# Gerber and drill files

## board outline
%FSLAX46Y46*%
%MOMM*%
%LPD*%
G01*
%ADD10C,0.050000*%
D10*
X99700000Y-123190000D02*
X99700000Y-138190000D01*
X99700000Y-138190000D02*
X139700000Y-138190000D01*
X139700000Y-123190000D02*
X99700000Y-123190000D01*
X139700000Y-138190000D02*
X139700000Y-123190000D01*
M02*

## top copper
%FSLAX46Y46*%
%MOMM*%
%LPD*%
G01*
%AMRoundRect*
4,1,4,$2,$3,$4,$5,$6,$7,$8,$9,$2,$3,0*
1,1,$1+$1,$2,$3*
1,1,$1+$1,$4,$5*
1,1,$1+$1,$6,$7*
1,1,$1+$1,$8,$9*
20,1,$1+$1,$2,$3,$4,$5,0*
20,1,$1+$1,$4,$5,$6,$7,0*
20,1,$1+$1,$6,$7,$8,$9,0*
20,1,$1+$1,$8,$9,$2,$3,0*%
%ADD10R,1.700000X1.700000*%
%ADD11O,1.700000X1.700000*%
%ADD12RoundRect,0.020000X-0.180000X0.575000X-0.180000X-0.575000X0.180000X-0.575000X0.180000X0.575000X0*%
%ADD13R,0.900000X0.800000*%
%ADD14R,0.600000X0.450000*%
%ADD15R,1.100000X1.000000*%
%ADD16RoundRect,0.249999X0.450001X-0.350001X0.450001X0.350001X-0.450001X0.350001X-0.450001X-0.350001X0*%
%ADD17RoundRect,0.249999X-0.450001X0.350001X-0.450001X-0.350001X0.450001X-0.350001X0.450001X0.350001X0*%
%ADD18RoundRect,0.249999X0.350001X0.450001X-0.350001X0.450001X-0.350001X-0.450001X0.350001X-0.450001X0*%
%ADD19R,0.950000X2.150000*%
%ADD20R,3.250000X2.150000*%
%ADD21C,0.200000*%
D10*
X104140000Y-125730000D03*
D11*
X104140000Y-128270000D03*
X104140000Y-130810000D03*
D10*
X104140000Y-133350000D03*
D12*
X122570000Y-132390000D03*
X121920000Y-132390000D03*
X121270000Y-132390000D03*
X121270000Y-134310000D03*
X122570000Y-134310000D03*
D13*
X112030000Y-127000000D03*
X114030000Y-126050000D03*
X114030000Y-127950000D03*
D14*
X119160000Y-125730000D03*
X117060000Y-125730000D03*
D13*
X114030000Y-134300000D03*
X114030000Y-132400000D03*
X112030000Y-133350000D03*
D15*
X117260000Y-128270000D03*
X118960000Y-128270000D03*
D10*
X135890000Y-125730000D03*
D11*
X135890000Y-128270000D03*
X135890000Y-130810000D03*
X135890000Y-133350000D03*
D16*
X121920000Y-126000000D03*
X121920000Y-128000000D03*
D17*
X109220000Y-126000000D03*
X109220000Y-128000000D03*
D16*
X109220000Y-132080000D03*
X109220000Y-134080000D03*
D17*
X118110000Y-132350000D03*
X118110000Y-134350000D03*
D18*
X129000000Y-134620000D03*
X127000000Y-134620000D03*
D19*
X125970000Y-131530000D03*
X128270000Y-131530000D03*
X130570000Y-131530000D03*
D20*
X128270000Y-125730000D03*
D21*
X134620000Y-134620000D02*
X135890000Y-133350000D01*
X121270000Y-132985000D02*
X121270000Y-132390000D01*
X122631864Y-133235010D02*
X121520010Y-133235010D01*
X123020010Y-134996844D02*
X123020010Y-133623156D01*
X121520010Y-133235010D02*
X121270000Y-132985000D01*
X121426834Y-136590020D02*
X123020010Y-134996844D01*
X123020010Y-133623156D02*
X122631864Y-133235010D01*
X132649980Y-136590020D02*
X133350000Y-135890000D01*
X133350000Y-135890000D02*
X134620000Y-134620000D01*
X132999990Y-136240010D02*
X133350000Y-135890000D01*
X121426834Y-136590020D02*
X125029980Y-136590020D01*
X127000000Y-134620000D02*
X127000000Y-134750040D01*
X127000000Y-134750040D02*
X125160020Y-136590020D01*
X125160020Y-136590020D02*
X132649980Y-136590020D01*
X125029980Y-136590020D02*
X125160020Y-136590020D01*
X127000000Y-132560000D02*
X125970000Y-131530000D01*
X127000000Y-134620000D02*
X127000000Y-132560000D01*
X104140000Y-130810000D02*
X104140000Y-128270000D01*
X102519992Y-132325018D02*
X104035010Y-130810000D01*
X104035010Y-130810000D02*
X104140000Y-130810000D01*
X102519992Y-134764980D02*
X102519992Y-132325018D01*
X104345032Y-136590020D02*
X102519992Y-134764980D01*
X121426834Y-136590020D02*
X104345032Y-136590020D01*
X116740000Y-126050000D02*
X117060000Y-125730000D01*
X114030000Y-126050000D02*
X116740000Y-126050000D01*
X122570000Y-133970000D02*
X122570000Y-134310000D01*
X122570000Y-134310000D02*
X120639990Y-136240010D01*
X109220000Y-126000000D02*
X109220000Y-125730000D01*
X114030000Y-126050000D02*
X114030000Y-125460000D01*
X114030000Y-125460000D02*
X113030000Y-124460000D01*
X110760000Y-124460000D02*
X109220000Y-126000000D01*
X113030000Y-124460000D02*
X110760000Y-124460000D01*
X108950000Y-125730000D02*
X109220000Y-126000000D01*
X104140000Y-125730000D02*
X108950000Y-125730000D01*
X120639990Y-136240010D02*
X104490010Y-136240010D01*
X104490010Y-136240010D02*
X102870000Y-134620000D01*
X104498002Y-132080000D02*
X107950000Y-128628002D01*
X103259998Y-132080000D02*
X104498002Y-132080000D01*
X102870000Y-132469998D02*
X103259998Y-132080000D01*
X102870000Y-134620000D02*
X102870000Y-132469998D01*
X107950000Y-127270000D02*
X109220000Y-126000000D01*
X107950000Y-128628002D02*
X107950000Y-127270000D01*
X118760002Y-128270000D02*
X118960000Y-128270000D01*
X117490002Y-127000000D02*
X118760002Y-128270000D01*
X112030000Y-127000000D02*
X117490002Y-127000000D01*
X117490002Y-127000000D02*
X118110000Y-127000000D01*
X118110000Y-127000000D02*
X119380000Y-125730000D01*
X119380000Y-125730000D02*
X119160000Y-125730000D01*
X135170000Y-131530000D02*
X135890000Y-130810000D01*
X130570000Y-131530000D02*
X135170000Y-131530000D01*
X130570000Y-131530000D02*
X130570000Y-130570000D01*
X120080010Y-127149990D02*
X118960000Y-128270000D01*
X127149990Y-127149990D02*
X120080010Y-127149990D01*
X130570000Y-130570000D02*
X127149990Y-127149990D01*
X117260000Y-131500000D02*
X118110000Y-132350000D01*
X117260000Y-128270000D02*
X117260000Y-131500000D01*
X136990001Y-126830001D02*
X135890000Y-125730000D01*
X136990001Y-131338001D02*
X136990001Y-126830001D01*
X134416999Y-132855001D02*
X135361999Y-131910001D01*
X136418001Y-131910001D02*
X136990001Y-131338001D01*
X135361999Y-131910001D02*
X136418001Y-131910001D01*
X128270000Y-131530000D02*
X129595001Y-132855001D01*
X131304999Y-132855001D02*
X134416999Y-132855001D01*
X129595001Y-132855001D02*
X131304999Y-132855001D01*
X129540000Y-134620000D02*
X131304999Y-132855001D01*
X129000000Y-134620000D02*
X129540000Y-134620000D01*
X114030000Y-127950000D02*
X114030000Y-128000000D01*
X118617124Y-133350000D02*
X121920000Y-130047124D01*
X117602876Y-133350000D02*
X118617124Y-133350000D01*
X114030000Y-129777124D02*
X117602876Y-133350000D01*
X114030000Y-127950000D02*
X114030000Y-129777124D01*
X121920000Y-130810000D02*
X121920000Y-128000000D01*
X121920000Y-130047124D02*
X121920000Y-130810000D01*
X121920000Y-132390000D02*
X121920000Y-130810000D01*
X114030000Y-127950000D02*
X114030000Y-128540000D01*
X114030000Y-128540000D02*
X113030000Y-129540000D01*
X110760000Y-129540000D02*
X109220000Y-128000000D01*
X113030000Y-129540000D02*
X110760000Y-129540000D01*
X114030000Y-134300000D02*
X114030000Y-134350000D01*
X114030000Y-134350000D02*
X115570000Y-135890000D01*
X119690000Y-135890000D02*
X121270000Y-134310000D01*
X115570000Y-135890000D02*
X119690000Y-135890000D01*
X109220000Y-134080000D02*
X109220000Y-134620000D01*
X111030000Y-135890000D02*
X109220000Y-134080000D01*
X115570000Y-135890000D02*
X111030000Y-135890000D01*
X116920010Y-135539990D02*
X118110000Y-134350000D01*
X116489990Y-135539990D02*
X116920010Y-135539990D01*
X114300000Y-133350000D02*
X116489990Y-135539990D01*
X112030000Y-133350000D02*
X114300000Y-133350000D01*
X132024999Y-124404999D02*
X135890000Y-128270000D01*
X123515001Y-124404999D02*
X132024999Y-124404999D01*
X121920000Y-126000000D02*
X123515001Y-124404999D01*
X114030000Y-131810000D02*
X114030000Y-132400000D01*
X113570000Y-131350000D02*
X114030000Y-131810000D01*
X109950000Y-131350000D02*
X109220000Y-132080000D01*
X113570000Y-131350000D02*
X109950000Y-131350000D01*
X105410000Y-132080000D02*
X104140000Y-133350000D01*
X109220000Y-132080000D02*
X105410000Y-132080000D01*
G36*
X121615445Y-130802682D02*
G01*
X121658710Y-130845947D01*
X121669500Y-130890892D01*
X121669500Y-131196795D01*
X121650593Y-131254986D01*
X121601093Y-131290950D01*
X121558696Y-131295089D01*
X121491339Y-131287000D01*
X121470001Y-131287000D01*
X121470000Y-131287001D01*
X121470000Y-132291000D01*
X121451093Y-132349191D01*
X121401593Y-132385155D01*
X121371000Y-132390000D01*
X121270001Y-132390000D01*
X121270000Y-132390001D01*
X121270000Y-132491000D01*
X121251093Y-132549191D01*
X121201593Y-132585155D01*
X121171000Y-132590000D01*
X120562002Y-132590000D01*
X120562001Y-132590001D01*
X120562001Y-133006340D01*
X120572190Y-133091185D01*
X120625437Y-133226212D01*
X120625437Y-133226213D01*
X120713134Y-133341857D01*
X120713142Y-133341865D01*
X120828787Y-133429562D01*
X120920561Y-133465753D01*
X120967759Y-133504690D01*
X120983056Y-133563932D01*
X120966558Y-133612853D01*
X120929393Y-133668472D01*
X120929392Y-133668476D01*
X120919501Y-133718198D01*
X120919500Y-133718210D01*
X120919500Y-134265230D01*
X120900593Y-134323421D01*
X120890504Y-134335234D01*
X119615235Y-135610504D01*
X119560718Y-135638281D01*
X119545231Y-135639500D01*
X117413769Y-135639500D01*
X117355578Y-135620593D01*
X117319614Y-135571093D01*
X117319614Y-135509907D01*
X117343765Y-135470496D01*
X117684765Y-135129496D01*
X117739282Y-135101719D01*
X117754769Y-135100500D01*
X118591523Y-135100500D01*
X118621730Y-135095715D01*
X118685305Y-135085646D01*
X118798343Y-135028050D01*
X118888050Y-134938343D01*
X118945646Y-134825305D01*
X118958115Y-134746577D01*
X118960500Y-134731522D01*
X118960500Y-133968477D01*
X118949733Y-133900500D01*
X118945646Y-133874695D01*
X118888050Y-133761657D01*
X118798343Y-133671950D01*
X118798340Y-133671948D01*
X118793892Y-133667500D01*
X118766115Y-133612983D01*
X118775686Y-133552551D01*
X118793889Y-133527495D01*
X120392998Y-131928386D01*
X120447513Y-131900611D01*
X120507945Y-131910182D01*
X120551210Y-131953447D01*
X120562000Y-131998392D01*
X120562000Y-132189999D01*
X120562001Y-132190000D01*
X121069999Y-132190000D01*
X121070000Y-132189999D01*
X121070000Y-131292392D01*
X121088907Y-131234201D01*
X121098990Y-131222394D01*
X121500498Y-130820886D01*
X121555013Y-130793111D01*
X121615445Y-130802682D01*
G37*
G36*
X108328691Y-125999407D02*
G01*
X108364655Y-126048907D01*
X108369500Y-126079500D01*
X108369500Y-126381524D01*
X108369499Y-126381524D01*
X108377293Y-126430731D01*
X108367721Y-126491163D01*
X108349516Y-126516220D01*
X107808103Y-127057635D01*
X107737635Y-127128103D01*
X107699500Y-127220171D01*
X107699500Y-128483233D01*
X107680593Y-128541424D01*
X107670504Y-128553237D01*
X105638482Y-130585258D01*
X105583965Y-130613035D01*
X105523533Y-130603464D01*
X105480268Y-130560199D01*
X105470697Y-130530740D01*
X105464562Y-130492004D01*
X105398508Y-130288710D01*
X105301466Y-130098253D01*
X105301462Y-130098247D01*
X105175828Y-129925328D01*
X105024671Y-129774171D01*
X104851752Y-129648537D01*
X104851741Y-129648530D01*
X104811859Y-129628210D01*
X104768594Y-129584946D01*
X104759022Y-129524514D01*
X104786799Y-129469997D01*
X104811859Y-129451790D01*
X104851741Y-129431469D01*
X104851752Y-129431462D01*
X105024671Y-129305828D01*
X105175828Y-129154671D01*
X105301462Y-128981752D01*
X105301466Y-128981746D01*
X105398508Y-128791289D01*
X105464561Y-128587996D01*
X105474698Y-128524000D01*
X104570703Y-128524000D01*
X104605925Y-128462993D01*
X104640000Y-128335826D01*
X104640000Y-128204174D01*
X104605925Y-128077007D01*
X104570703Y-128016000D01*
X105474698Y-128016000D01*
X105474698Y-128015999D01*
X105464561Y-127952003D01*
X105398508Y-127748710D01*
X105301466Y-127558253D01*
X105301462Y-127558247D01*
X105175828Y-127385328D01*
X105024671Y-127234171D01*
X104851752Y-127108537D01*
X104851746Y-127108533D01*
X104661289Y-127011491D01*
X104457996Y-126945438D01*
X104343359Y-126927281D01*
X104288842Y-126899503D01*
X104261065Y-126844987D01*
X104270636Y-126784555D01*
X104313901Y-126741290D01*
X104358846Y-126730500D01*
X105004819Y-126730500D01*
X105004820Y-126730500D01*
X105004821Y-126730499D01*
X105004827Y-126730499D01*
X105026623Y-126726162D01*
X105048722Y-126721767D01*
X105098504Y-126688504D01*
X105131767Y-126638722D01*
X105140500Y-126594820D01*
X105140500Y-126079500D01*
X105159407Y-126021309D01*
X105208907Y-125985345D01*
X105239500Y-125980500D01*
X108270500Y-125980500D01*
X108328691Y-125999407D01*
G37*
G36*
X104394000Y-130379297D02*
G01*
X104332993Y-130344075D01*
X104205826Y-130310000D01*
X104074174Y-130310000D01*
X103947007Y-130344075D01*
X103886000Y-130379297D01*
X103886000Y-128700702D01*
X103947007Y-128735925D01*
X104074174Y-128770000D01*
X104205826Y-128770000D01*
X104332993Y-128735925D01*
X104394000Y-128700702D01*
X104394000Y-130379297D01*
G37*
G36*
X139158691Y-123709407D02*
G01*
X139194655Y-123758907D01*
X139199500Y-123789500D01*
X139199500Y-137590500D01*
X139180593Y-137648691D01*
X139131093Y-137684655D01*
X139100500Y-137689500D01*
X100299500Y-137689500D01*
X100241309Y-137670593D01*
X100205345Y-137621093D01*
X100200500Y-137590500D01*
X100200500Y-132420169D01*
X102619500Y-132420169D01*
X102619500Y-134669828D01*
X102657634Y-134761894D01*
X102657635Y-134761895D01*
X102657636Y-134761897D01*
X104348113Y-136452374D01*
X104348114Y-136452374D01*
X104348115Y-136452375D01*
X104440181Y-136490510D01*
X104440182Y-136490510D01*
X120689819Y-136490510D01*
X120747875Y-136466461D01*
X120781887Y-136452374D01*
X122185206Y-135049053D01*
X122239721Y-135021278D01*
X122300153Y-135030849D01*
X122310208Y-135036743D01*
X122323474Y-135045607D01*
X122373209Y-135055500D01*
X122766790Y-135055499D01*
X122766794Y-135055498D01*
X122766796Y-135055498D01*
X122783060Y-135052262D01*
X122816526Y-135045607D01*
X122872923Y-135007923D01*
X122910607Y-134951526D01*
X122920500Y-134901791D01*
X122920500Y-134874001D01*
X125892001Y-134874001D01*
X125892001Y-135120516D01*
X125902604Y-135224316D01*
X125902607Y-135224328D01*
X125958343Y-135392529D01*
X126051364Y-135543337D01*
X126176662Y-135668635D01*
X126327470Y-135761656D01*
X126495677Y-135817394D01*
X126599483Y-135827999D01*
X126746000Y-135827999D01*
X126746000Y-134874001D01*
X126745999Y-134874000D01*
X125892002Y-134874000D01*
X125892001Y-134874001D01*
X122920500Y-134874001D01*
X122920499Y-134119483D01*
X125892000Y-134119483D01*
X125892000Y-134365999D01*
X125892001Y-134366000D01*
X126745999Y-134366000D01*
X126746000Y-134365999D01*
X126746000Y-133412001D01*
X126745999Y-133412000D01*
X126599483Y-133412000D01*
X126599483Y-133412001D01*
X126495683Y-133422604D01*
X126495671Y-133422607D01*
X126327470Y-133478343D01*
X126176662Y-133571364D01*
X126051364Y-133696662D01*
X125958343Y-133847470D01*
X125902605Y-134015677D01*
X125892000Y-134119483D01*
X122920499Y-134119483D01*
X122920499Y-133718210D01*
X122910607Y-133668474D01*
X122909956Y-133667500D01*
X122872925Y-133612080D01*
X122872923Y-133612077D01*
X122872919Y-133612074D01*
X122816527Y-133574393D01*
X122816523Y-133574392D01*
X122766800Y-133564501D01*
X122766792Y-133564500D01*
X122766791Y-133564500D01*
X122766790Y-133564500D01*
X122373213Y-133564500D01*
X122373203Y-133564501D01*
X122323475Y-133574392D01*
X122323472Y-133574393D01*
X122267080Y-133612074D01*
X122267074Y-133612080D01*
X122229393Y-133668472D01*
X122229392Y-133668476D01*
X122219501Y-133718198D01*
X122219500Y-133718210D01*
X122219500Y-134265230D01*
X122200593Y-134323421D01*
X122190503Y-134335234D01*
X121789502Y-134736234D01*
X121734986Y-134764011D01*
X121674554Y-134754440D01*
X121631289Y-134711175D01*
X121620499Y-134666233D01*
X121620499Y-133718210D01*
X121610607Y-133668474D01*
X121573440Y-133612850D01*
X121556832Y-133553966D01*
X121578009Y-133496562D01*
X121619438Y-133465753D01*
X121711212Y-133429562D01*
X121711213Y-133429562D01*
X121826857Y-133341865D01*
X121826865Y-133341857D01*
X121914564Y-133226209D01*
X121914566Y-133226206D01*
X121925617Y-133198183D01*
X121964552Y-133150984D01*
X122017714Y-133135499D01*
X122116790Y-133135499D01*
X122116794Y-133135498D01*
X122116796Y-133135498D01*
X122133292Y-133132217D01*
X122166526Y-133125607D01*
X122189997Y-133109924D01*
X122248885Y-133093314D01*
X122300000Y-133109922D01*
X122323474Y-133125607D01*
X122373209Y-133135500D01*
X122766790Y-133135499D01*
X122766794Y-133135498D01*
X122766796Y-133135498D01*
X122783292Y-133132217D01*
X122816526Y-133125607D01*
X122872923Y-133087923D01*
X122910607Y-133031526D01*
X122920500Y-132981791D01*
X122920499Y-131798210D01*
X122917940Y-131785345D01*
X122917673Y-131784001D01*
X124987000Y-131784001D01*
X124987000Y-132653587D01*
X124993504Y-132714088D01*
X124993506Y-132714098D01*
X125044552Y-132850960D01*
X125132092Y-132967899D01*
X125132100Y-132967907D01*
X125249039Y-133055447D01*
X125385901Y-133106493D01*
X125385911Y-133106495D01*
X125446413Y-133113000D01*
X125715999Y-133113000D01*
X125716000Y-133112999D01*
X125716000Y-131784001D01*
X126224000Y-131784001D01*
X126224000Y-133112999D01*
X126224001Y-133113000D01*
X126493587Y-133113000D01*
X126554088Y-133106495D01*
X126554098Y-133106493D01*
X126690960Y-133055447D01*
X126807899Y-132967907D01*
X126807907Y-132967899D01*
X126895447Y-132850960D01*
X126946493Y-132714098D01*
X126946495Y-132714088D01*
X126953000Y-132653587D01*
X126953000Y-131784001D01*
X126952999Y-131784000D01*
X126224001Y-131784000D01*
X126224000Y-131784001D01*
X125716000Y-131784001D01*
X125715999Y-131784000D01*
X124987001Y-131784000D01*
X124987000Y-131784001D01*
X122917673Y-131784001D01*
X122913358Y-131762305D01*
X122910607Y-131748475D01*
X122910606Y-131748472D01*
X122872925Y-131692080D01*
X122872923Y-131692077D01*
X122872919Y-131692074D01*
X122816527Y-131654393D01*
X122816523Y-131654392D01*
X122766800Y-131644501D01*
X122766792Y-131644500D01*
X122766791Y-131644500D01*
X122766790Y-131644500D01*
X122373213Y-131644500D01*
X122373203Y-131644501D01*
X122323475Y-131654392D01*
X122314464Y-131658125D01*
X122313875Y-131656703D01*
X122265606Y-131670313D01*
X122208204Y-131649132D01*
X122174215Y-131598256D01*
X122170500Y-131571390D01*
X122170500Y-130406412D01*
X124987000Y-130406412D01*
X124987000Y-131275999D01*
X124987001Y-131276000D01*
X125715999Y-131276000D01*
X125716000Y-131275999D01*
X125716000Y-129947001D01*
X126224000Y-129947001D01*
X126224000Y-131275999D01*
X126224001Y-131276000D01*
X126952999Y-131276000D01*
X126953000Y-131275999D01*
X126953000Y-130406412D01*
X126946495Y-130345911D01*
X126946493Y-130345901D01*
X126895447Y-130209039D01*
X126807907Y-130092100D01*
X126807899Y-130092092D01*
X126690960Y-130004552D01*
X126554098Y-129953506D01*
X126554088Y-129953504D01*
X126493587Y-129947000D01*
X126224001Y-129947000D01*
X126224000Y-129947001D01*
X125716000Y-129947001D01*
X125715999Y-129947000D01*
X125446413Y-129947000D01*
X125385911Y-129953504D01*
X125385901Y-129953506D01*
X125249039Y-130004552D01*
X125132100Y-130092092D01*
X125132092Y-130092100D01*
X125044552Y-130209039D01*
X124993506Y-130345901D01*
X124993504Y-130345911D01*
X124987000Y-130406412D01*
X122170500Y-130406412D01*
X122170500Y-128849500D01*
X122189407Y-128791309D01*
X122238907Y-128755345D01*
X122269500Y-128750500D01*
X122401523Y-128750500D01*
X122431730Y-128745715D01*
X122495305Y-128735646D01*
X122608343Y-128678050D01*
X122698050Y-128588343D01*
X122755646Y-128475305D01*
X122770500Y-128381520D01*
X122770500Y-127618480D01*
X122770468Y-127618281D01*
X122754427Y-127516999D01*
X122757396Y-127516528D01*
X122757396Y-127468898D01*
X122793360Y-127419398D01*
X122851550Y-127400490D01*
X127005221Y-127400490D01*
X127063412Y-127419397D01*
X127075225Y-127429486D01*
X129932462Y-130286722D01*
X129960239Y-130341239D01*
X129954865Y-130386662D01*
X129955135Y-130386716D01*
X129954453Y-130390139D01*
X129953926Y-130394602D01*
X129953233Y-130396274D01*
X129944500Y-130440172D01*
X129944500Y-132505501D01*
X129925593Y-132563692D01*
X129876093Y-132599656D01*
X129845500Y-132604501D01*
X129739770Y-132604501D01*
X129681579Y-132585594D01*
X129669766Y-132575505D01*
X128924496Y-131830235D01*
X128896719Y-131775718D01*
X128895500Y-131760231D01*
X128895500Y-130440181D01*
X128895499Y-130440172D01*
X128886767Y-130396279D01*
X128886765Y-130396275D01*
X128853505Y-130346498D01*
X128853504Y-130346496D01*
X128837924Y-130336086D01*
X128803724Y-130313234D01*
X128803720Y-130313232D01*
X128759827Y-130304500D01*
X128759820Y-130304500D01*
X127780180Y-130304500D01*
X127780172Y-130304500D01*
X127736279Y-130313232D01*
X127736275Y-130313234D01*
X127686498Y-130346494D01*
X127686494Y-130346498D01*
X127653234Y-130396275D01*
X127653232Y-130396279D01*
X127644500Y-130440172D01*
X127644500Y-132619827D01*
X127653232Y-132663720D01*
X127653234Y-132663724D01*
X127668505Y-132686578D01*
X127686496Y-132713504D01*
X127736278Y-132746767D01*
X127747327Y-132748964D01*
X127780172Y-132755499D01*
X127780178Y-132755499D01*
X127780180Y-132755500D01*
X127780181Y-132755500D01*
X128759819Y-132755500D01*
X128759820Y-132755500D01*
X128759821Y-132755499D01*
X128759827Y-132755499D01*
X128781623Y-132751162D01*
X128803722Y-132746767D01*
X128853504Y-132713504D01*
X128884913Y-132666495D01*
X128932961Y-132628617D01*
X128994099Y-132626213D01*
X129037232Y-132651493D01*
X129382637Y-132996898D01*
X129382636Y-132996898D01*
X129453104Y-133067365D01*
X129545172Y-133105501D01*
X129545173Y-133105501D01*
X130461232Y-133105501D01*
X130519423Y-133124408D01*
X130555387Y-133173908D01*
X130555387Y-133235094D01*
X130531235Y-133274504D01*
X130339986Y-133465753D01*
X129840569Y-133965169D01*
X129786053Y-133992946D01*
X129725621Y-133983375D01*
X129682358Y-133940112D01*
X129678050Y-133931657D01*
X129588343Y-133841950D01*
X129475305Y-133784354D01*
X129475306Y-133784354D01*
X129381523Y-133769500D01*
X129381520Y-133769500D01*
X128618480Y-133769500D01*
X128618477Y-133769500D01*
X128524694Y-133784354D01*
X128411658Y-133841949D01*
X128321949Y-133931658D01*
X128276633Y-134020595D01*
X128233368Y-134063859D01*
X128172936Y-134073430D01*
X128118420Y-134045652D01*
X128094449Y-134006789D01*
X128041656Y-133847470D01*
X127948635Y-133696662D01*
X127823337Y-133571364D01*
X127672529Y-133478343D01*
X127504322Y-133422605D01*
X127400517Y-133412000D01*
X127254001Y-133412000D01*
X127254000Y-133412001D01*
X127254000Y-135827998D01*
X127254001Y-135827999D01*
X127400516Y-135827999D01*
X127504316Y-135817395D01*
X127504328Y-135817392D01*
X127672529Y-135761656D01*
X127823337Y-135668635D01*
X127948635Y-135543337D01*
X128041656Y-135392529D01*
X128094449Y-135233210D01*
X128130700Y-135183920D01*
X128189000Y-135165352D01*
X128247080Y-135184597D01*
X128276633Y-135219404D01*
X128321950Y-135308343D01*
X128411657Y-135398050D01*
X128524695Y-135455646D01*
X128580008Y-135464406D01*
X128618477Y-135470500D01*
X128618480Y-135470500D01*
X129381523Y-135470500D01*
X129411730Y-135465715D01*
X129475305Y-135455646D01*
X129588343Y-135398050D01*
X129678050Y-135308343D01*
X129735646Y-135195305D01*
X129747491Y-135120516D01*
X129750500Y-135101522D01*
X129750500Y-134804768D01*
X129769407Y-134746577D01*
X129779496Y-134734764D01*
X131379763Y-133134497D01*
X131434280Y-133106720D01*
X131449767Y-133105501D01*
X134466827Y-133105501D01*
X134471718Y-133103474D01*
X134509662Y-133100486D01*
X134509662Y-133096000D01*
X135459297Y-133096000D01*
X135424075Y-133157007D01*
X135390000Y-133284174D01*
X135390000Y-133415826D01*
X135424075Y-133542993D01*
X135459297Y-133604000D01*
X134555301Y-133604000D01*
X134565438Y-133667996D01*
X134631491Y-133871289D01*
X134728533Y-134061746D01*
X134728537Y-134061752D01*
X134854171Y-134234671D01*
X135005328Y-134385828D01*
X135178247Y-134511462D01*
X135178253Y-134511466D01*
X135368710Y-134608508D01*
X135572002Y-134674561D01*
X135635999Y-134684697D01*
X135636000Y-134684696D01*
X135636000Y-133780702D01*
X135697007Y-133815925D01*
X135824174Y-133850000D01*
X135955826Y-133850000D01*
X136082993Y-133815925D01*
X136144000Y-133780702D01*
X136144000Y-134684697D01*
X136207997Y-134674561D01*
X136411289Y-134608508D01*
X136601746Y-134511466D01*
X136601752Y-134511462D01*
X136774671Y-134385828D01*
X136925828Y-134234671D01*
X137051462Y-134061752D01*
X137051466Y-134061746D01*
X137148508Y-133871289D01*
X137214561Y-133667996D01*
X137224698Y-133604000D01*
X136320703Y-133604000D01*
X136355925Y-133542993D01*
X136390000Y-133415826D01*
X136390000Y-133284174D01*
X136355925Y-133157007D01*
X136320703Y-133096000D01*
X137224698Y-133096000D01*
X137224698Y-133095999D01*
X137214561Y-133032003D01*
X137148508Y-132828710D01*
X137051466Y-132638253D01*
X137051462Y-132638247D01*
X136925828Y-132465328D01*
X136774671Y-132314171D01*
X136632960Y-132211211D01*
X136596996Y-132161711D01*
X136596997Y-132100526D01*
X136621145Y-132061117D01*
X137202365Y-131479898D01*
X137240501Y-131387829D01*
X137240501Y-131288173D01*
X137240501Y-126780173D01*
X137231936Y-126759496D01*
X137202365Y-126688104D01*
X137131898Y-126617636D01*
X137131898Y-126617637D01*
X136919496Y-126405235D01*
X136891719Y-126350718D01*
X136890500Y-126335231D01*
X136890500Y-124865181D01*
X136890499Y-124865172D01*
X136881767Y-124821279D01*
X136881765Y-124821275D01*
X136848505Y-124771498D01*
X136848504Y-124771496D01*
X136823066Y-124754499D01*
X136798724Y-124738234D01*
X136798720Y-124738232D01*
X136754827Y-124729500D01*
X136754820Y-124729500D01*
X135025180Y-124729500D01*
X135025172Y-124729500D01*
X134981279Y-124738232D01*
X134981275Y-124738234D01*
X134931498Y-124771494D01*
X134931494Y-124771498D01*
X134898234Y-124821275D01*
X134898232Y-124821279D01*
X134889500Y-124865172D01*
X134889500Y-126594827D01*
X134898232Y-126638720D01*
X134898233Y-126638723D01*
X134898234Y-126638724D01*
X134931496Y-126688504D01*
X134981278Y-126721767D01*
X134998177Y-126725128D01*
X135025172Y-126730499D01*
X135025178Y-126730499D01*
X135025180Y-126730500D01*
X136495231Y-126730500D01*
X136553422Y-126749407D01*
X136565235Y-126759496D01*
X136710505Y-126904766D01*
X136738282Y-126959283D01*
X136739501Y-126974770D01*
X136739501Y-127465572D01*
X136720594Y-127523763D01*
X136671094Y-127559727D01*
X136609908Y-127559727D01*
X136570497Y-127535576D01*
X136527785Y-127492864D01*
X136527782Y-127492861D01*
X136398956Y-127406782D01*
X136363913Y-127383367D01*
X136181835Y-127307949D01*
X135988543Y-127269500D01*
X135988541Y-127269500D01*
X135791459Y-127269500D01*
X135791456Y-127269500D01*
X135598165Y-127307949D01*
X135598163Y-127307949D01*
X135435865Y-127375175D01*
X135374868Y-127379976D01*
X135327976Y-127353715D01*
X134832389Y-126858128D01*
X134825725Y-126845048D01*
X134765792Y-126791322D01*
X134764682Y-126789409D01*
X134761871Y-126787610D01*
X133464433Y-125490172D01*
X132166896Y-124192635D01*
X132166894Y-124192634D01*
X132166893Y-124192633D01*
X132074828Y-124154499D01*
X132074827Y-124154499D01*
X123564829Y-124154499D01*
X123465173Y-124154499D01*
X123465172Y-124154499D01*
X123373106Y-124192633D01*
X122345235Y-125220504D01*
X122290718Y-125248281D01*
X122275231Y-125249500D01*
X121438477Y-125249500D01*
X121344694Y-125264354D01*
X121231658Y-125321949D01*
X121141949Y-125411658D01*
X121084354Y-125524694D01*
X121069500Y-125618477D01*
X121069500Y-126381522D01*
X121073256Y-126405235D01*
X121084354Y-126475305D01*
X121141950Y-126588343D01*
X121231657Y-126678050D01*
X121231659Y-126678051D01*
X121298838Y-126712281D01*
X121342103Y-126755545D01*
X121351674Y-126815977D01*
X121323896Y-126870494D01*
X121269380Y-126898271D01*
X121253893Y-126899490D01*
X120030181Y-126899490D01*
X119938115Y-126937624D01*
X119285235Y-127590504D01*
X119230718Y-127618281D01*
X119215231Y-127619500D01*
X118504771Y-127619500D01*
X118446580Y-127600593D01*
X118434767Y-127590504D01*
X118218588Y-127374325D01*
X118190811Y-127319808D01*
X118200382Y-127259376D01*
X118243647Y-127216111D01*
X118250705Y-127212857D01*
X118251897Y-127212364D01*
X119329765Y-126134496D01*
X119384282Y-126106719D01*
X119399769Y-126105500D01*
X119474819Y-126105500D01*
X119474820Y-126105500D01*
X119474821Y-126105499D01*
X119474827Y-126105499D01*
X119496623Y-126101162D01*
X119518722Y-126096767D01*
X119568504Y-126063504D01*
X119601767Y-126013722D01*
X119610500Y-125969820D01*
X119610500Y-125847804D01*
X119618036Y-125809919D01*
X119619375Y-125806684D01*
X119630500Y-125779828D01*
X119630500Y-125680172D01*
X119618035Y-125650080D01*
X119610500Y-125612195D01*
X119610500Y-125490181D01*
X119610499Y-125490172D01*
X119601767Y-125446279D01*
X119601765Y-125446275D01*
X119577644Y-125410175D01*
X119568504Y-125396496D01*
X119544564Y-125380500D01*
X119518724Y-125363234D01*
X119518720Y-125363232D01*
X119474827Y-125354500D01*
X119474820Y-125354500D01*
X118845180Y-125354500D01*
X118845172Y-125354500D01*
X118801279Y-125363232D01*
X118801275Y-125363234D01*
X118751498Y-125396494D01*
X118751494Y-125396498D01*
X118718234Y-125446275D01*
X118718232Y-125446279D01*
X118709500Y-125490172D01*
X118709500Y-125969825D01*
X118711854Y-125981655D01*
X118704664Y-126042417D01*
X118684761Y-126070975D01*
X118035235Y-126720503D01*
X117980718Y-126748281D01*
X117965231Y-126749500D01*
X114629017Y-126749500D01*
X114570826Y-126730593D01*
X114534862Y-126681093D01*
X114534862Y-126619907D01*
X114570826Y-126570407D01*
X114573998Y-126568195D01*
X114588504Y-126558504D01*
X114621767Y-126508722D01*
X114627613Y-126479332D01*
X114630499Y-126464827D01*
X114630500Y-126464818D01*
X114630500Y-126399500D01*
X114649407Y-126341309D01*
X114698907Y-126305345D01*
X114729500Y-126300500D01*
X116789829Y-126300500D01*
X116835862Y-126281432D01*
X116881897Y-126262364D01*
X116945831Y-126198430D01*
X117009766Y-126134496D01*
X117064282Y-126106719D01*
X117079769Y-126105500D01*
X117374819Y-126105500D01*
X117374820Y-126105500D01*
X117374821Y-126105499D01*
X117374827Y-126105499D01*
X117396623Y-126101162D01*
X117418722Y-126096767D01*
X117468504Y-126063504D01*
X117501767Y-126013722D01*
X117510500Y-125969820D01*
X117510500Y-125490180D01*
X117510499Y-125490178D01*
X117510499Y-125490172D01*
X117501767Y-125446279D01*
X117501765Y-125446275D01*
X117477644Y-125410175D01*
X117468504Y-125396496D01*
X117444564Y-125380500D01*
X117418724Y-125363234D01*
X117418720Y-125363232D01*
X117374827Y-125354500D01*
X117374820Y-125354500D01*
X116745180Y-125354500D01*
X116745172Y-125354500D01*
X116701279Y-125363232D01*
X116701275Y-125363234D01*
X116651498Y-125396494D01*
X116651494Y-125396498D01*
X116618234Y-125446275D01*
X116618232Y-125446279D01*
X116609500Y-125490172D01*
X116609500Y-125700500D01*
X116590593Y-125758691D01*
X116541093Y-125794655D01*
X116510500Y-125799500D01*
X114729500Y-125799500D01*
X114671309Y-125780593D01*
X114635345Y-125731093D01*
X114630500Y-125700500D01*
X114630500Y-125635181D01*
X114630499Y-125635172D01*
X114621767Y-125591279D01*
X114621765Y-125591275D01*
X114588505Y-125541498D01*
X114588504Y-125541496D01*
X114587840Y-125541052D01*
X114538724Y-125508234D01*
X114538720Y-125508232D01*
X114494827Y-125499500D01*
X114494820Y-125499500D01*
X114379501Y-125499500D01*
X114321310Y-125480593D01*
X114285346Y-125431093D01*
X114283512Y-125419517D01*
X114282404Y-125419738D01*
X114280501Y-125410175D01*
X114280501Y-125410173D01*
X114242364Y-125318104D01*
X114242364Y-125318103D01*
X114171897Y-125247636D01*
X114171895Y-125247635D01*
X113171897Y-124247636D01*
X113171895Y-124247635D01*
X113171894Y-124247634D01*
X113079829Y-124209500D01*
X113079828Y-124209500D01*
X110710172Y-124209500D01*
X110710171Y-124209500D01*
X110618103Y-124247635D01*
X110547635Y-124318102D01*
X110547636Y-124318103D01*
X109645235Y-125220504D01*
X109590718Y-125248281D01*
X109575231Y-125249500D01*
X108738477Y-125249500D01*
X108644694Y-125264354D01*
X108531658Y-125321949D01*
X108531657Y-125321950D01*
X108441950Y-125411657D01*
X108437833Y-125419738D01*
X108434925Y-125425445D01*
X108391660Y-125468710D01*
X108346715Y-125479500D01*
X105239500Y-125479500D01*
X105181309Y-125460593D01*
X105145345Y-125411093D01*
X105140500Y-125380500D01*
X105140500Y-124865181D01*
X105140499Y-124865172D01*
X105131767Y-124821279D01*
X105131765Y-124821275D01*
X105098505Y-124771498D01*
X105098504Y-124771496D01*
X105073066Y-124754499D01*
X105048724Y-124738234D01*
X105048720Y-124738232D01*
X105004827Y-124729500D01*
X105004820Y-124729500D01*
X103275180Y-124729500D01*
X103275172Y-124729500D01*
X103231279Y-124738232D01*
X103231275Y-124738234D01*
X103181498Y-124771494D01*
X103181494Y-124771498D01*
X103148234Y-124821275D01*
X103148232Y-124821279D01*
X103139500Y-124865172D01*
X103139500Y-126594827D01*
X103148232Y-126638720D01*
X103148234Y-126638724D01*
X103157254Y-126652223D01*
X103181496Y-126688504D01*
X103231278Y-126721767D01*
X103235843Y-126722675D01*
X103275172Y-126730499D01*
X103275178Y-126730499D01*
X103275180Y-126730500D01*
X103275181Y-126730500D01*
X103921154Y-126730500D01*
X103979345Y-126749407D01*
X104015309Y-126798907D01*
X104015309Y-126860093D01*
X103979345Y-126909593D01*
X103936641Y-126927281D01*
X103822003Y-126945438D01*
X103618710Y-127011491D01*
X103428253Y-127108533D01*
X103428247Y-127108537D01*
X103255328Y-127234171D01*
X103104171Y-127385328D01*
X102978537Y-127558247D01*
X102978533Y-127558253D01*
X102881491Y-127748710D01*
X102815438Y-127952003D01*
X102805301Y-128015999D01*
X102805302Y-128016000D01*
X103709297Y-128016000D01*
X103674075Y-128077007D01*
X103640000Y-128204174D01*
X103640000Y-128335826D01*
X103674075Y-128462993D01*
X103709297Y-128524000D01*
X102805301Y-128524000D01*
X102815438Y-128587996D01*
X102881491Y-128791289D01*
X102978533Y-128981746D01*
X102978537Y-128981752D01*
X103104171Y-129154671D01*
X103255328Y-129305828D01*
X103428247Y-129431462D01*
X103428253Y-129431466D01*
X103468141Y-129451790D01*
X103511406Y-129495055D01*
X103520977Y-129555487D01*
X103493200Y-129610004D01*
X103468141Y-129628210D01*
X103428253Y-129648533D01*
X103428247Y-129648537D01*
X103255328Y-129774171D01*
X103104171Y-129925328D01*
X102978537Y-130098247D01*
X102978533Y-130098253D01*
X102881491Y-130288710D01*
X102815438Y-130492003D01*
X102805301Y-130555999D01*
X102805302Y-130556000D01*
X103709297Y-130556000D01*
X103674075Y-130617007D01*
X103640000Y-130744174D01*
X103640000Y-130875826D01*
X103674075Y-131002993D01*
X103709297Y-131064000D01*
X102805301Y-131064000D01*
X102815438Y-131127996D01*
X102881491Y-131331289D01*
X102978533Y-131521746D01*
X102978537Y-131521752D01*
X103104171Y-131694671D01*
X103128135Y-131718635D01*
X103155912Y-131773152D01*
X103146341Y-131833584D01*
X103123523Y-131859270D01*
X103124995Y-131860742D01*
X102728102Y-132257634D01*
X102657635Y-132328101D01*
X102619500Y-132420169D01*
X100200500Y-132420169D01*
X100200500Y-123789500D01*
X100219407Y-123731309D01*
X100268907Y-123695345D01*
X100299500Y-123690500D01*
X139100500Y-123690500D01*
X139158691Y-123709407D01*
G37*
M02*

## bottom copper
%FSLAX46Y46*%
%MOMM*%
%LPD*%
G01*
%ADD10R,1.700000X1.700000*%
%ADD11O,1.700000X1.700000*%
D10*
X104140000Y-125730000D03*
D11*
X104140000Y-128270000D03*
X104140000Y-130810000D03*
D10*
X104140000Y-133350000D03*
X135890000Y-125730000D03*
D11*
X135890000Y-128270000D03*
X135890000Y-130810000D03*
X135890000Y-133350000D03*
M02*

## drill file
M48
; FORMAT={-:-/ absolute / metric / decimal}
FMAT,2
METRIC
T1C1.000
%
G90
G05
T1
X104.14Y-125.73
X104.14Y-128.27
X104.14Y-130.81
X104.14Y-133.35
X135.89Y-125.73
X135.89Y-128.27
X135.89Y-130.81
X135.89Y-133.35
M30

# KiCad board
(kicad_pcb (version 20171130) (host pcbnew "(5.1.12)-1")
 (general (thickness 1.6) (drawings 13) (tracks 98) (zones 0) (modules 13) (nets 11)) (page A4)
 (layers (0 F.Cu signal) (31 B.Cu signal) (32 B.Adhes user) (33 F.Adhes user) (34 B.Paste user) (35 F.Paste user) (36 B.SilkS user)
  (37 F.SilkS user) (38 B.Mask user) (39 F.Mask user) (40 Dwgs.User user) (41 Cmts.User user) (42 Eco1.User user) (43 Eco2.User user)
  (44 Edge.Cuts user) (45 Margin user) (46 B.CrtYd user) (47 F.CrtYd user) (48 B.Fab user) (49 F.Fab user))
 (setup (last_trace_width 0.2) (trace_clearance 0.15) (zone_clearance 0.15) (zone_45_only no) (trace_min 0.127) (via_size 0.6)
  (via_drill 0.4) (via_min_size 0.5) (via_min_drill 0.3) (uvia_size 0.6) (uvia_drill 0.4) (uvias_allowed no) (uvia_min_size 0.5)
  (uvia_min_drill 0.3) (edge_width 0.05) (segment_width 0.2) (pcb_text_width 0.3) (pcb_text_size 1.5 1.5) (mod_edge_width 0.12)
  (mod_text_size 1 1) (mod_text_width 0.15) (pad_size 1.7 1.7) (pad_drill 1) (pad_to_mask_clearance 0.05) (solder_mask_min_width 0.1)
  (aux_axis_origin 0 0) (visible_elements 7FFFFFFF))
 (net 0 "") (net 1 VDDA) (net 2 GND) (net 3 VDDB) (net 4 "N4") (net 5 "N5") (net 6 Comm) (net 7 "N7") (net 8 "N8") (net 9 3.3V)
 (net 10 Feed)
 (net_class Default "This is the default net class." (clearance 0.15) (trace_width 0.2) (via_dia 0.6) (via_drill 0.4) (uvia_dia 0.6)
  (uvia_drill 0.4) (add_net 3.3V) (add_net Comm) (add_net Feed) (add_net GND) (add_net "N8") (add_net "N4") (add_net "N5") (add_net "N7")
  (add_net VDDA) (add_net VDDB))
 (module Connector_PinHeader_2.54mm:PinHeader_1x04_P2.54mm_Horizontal (layer F.Cu) (at 104.14 133.35 180)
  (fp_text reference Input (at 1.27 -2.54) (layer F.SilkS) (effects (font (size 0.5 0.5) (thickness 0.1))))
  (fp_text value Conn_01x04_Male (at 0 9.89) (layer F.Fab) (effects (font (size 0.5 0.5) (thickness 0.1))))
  (pad 4 thru_hole rect (at 0 7.62 180) (size 1.7 1.7) (drill 1) (layers *.Cu *.Mask) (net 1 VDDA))
  (pad 3 thru_hole oval (at 0 5.08 180) (size 1.7 1.7) (drill 1) (layers *.Cu *.Mask) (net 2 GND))
  (pad 2 thru_hole oval (at 0 2.54 180) (size 1.7 1.7) (drill 1) (layers *.Cu *.Mask) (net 2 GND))
  (pad 1 thru_hole rect (at 0 0 180) (size 1.7 1.7) (drill 1) (layers *.Cu *.Mask) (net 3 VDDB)))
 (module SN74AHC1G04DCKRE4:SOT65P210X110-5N (layer F.Cu) (at 121.92 133.35 270)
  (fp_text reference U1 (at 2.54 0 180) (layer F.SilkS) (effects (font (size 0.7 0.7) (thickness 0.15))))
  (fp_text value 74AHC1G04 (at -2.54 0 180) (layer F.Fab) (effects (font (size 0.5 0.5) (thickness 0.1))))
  (pad 1 smd roundrect (at -0.96 -0.65 270) (size 1.19 0.4) (layers F.Cu F.Paste F.Mask) (roundrect_rratio 0.05))
  (pad 2 smd roundrect (at -0.96 0 270) (size 1.19 0.4) (layers F.Cu F.Paste F.Mask) (roundrect_rratio 0.05) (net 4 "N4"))
  (pad 3 smd roundrect (at -0.96 0.65 270) (size 1.19 0.4) (layers F.Cu F.Paste F.Mask) (roundrect_rratio 0.05) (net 2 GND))
  (pad 4 smd roundrect (at 0.96 0.65 270) (size 1.19 0.4) (layers F.Cu F.Paste F.Mask) (roundrect_rratio 0.05) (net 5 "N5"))
  (pad 5 smd roundrect (at 0.96 -0.65 270) (size 1.19 0.4) (layers F.Cu F.Paste F.Mask) (roundrect_rratio 0.05) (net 1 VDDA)))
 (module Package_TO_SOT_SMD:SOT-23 (layer F.Cu) (at 113.03 127 180)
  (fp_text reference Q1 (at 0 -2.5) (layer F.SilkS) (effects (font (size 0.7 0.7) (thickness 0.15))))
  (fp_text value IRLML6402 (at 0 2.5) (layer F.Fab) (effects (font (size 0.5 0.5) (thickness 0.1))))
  (pad 3 smd rect (at 1 0 180) (size 0.9 0.8) (layers F.Cu F.Paste F.Mask) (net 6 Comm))
  (pad 2 smd rect (at -1 0.95 180) (size 0.9 0.8) (layers F.Cu F.Paste F.Mask) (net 1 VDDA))
  (pad 1 smd rect (at -1 -0.95 180) (size 0.9 0.8) (layers F.Cu F.Paste F.Mask) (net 4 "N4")))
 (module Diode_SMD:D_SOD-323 (layer F.Cu) (at 118.11 125.73 180)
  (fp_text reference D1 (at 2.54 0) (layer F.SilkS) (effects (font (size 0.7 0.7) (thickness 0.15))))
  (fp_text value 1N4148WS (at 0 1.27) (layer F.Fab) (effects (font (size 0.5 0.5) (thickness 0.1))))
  (pad 1 smd rect (at -1.05 0 180) (size 0.6 0.45) (layers F.Cu F.Paste F.Mask) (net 6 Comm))
  (pad 2 smd rect (at 1.05 0 180) (size 0.6 0.45) (layers F.Cu F.Paste F.Mask) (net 1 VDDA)))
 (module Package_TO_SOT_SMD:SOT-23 (layer F.Cu) (at 113.03 133.35 180)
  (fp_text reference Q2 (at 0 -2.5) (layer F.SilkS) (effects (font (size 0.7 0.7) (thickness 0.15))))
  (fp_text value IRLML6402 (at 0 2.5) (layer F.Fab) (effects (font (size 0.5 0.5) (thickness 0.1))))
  (pad 1 smd rect (at -1 -0.95 180) (size 0.9 0.8) (layers F.Cu F.Paste F.Mask) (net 5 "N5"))
  (pad 2 smd rect (at -1 0.95 180) (size 0.9 0.8) (layers F.Cu F.Paste F.Mask) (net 3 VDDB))
  (pad 3 smd rect (at 1 0 180) (size 0.9 0.8) (layers F.Cu F.Paste F.Mask) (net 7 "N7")))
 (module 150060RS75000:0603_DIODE (layer F.Cu) (at 118.11 128.27)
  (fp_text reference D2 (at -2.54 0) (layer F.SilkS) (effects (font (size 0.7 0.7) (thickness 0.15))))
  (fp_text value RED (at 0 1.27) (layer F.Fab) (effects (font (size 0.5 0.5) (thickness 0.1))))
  (pad 2 smd rect (at -0.85 0) (size 1.1 1) (layers F.Cu F.Paste F.Mask) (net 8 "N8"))
  (pad 1 smd rect (at 0.85 0) (size 1.1 1) (layers F.Cu F.Paste F.Mask) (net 6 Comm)))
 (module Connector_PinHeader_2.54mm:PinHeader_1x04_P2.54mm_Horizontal (layer F.Cu) (at 135.89 125.73)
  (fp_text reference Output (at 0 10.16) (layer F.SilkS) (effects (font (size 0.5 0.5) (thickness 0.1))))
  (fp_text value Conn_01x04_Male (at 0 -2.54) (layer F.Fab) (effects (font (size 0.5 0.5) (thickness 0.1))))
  (pad 1 thru_hole rect (at 0 0) (size 1.7 1.7) (drill 1) (layers *.Cu *.Mask) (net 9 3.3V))
  (pad 2 thru_hole oval (at 0 2.54) (size 1.7 1.7) (drill 1) (layers *.Cu *.Mask) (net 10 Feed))
  (pad 3 thru_hole oval (at 0 5.08) (size 1.7 1.7) (drill 1) (layers *.Cu *.Mask) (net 6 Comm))
  (pad 4 thru_hole oval (at 0 7.62) (size 1.7 1.7) (drill 1) (layers *.Cu *.Mask) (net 2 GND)))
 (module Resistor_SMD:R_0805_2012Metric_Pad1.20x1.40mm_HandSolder (layer F.Cu) (at 121.92 127 90)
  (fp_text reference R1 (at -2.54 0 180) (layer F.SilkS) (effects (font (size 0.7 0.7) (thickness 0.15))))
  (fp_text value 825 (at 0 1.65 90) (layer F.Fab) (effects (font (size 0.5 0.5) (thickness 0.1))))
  (pad 2 smd roundrect (at 1 0 90) (size 1.2 1.4) (layers F.Cu F.Paste F.Mask) (roundrect_rratio 0.2083325) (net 10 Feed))
  (pad 1 smd roundrect (at -1 0 90) (size 1.2 1.4) (layers F.Cu F.Paste F.Mask) (roundrect_rratio 0.2083325) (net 4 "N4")))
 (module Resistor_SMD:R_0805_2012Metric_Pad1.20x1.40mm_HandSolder (layer F.Cu) (at 109.22 127 270)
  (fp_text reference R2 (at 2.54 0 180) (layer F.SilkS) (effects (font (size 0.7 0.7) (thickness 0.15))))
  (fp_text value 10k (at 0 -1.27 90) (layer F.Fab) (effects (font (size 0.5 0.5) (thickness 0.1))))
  (pad 1 smd roundrect (at -1 0 270) (size 1.2 1.4) (layers F.Cu F.Paste F.Mask) (roundrect_rratio 0.2083325) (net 1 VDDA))
  (pad 2 smd roundrect (at 1 0 270) (size 1.2 1.4) (layers F.Cu F.Paste F.Mask) (roundrect_rratio 0.2083325) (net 4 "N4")))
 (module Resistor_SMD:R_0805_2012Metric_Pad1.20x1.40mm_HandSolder (layer F.Cu) (at 109.22 133.08 90)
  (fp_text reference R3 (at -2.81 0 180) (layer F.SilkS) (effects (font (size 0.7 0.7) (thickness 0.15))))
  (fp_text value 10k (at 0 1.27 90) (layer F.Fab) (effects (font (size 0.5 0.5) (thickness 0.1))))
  (pad 2 smd roundrect (at 1 0 90) (size 1.2 1.4) (layers F.Cu F.Paste F.Mask) (roundrect_rratio 0.2083325) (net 3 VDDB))
  (pad 1 smd roundrect (at -1 0 90) (size 1.2 1.4) (layers F.Cu F.Paste F.Mask) (roundrect_rratio 0.2083325) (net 5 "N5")))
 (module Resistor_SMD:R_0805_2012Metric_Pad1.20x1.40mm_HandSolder (layer F.Cu) (at 118.11 133.35 270)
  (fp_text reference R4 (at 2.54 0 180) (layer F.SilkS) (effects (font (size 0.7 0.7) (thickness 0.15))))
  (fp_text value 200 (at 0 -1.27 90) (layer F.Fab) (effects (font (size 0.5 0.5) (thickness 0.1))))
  (pad 1 smd roundrect (at -1 0 270) (size 1.2 1.4) (layers F.Cu F.Paste F.Mask) (roundrect_rratio 0.2083325) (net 8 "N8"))
  (pad 2 smd roundrect (at 1 0 270) (size 1.2 1.4) (layers F.Cu F.Paste F.Mask) (roundrect_rratio 0.2083325) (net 7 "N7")))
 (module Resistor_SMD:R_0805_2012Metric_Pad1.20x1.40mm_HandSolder (layer F.Cu) (at 128 134.62 180)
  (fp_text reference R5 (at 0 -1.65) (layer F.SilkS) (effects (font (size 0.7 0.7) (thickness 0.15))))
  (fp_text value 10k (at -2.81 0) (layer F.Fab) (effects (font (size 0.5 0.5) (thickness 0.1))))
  (pad 1 smd roundrect (at -1 0 180) (size 1.2 1.4) (layers F.Cu F.Paste F.Mask) (roundrect_rratio 0.2083325) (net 9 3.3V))
  (pad 2 smd roundrect (at 1 0 180) (size 1.2 1.4) (layers F.Cu F.Paste F.Mask) (roundrect_rratio 0.2083325) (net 2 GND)))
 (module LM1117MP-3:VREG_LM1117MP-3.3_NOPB (layer F.Cu) (at 128.27 128.63 90)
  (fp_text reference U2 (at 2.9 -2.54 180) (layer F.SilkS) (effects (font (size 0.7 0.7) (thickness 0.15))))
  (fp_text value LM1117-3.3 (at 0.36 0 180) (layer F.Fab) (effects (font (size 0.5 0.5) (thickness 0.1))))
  (pad 1 smd rect (at -2.9 -2.3) (size 0.95 2.15) (layers F.Cu F.Paste F.Mask) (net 2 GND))
  (pad 2 smd rect (at -2.9 0) (size 0.95 2.15) (layers F.Cu F.Paste F.Mask) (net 9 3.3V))
  (pad 3 smd rect (at -2.9 2.3) (size 0.95 2.15) (layers F.Cu F.Paste F.Mask) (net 6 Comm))
  (pad 4 smd rect (at 2.9 0) (size 3.25 2.15) (layers F.Cu F.Paste F.Mask)))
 (gr_line (start 99.7 123.19) (end 99.7 138.19) (layer Edge.Cuts) (width 0.05))
 (gr_line (start 99.7 138.19) (end 139.7 138.19) (layer Edge.Cuts) (width 0.05))
 (gr_line (start 139.7 123.19) (end 99.7 123.19) (layer Edge.Cuts) (width 0.05))
 (gr_line (start 139.7 138.19) (end 139.7 123.19) (layer Edge.Cuts) (width 0.05))
 (segment (start 134.62 134.62) (end 135.89 133.35) (width 0.2) (layer F.Cu) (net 2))
 (segment (start 121.27 132.985) (end 121.27 132.39) (width 0.2) (layer F.Cu) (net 2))
 (segment (start 122.631864 133.23501) (end 121.52001 133.23501) (width 0.2) (layer F.Cu) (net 2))
 (segment (start 123.02001 134.996844) (end 123.02001 133.623156) (width 0.2) (layer F.Cu) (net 2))
 (segment (start 121.52001 133.23501) (end 121.27 132.985) (width 0.2) (layer F.Cu) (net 2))
 (segment (start 121.426834 136.59002) (end 123.02001 134.996844) (width 0.2) (layer F.Cu) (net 2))
 (segment (start 123.02001 133.623156) (end 122.631864 133.23501) (width 0.2) (layer F.Cu) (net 2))
 (segment (start 132.64998 136.59002) (end 133.35 135.89) (width 0.2) (layer F.Cu) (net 2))
 (segment (start 133.35 135.89) (end 134.62 134.62) (width 0.2) (layer F.Cu) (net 2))
 (segment (start 132.99999 136.24001) (end 133.35 135.89) (width 0.2) (layer F.Cu) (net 2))
 (segment (start 121.426834 136.59002) (end 125.02998 136.59002) (width 0.2) (layer F.Cu) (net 2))
 (segment (start 127 134.62) (end 127 134.75004) (width 0.2) (layer F.Cu) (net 2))
 (segment (start 127 134.75004) (end 125.16002 136.59002) (width 0.2) (layer F.Cu) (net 2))
 (segment (start 125.16002 136.59002) (end 132.64998 136.59002) (width 0.2) (layer F.Cu) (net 2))
 (segment (start 125.02998 136.59002) (end 125.16002 136.59002) (width 0.2) (layer F.Cu) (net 2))
 (segment (start 127 132.56) (end 125.97 131.53) (width 0.2) (layer F.Cu) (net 2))
 (segment (start 127 134.62) (end 127 132.56) (width 0.2) (layer F.Cu) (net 2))
 (segment (start 104.14 130.81) (end 104.14 128.27) (width 0.2) (layer F.Cu) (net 2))
 (segment (start 102.519992 132.325018) (end 104.03501 130.81) (width 0.2) (layer F.Cu) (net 2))
 (segment (start 104.03501 130.81) (end 104.14 130.81) (width 0.2) (layer F.Cu) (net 2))
 (segment (start 102.519992 134.76498) (end 102.519992 132.325018) (width 0.2) (layer F.Cu) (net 2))
 (segment (start 104.345032 136.59002) (end 102.519992 134.76498) (width 0.2) (layer F.Cu) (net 2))
 (segment (start 121.426834 136.59002) (end 104.345032 136.59002) (width 0.2) (layer F.Cu) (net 2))
 (segment (start 116.74 126.05) (end 117.06 125.73) (width 0.2) (layer F.Cu) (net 1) (status 20))
 (segment (start 114.03 126.05) (end 116.74 126.05) (width 0.2) (layer F.Cu) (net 1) (status 10))
 (segment (start 122.57 133.97) (end 122.57 134.31) (width 0.2) (layer F.Cu) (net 1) (status 30))
 (segment (start 122.57 134.31) (end 120.63999 136.24001) (width 0.2) (layer F.Cu) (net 1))
 (segment (start 109.22 126) (end 109.22 125.73) (width 0.2) (layer F.Cu) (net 1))
 (segment (start 114.03 126.05) (end 114.03 125.46) (width 0.2) (layer F.Cu) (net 1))
 (segment (start 114.03 125.46) (end 113.03 124.46) (width 0.2) (layer F.Cu) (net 1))
 (segment (start 110.76 124.46) (end 109.22 126) (width 0.2) (layer F.Cu) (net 1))
 (segment (start 113.03 124.46) (end 110.76 124.46) (width 0.2) (layer F.Cu) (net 1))
 (segment (start 108.95 125.73) (end 109.22 126) (width 0.2) (layer F.Cu) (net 1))
 (segment (start 104.14 125.73) (end 108.95 125.73) (width 0.2) (layer F.Cu) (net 1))
 (segment (start 120.63999 136.24001) (end 104.49001 136.24001) (width 0.2) (layer F.Cu) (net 1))
 (segment (start 104.49001 136.24001) (end 102.87 134.62) (width 0.2) (layer F.Cu) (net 1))
 (segment (start 104.498002 132.08) (end 107.95 128.628002) (width 0.2) (layer F.Cu) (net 1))
 (segment (start 103.259998 132.08) (end 104.498002 132.08) (width 0.2) (layer F.Cu) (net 1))
 (segment (start 102.87 132.469998) (end 103.259998 132.08) (width 0.2) (layer F.Cu) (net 1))
 (segment (start 102.87 134.62) (end 102.87 132.469998) (width 0.2) (layer F.Cu) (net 1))
 (segment (start 107.95 127.27) (end 109.22 126) (width 0.2) (layer F.Cu) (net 1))
 (segment (start 107.95 128.628002) (end 107.95 127.27) (width 0.2) (layer F.Cu) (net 1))
 (segment (start 118.760002 128.27) (end 118.96 128.27) (width 0.2) (layer F.Cu) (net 6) (status 30))
 (segment (start 117.490002 127) (end 118.760002 128.27) (width 0.2) (layer F.Cu) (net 6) (status 20))
 (segment (start 112.03 127) (end 117.490002 127) (width 0.2) (layer F.Cu) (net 6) (status 10))
 (segment (start 117.490002 127) (end 118.11 127) (width 0.2) (layer F.Cu) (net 6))
 (segment (start 118.11 127) (end 119.38 125.73) (width 0.2) (layer F.Cu) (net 6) (status 20))
 (segment (start 119.38 125.73) (end 119.16 125.73) (width 0.2) (layer F.Cu) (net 6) (status 30))
 (segment (start 135.17 131.53) (end 135.89 130.81) (width 0.2) (layer F.Cu) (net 6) (status 20))
 (segment (start 130.57 131.53) (end 135.17 131.53) (width 0.2) (layer F.Cu) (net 6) (status 10))
 (segment (start 130.57 131.53) (end 130.57 130.57) (width 0.2) (layer F.Cu) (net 6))
 (segment (start 120.08001 127.14999) (end 118.96 128.27) (width 0.2) (layer F.Cu) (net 6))
 (segment (start 127.14999 127.14999) (end 120.08001 127.14999) (width 0.2) (layer F.Cu) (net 6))
 (segment (start 130.57 130.57) (end 127.14999 127.14999) (width 0.2) (layer F.Cu) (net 6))
 (segment (start 117.26 131.5) (end 118.11 132.35) (width 0.2) (layer F.Cu) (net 8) (status 20))
 (segment (start 117.26 128.27) (end 117.26 131.5) (width 0.2) (layer F.Cu) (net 8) (status 10))
 (segment (start 136.990001 126.830001) (end 135.89 125.73) (width 0.2) (layer F.Cu) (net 9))
 (segment (start 136.990001 131.338001) (end 136.990001 126.830001) (width 0.2) (layer F.Cu) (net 9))
 (segment (start 134.416999 132.855001) (end 135.361999 131.910001) (width 0.2) (layer F.Cu) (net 9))
 (segment (start 136.418001 131.910001) (end 136.990001 131.338001) (width 0.2) (layer F.Cu) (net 9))
 (segment (start 135.361999 131.910001) (end 136.418001 131.910001) (width 0.2) (layer F.Cu) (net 9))
 (segment (start 128.27 131.53) (end 129.595001 132.855001) (width 0.2) (layer F.Cu) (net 9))
 (segment (start 131.304999 132.855001) (end 134.416999 132.855001) (width 0.2) (layer F.Cu) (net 9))
 (segment (start 129.595001 132.855001) (end 131.304999 132.855001) (width 0.2) (layer F.Cu) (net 9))
 (segment (start 129.54 134.62) (end 131.304999 132.855001) (width 0.2) (layer F.Cu) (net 9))
 (segment (start 129 134.62) (end 129.54 134.62) (width 0.2) (layer F.Cu) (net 9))
 (segment (start 114.03 127.95) (end 114.03 128) (width 0.2) (layer F.Cu) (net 4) (status 30))
 (segment (start 118.617124 133.35) (end 121.92 130.047124) (width 0.2) (layer F.Cu) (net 4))
 (segment (start 117.602876 133.35) (end 118.617124 133.35) (width 0.2) (layer F.Cu) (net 4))
 (segment (start 114.03 129.777124) (end 117.602876 133.35) (width 0.2) (layer F.Cu) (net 4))
 (segment (start 114.03 127.95) (end 114.03 129.777124) (width 0.2) (layer F.Cu) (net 4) (status 10))
 (segment (start 121.92 130.81) (end 121.92 128) (width 0.2) (layer F.Cu) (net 4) (status 20))
 (segment (start 121.92 130.047124) (end 121.92 130.81) (width 0.2) (layer F.Cu) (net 4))
 (segment (start 121.92 132.39) (end 121.92 130.81) (width 0.2) (layer F.Cu) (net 4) (status 10))
 (segment (start 114.03 127.95) (end 114.03 128.54) (width 0.2) (layer F.Cu) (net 4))
 (segment (start 114.03 128.54) (end 113.03 129.54) (width 0.2) (layer F.Cu) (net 4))
 (segment (start 110.76 129.54) (end 109.22 128) (width 0.2) (layer F.Cu) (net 4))
 (segment (start 113.03 129.54) (end 110.76 129.54) (width 0.2) (layer F.Cu) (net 4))
 (segment (start 114.03 134.3) (end 114.03 134.35) (width 0.2) (layer F.Cu) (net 5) (status 30))
 (segment (start 114.03 134.35) (end 115.57 135.89) (width 0.2) (layer F.Cu) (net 5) (status 10))
 (segment (start 119.69 135.89) (end 121.27 134.31) (width 0.2) (layer F.Cu) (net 5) (status 20))
 (segment (start 115.57 135.89) (end 119.69 135.89) (width 0.2) (layer F.Cu) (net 5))
 (segment (start 109.22 134.08) (end 109.22 134.62) (width 0.2) (layer F.Cu) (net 5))
 (segment (start 111.03 135.89) (end 109.22 134.08) (width 0.2) (layer F.Cu) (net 5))
 (segment (start 115.57 135.89) (end 111.03 135.89) (width 0.2) (layer F.Cu) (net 5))
 (segment (start 116.92001 135.53999) (end 118.11 134.35) (width 0.2) (layer F.Cu) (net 7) (status 20))
 (segment (start 116.48999 135.53999) (end 116.92001 135.53999) (width 0.2) (layer F.Cu) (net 7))
 (segment (start 114.3 133.35) (end 116.48999 135.53999) (width 0.2) (layer F.Cu) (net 7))
 (segment (start 112.03 133.35) (end 114.3 133.35) (width 0.2) (layer F.Cu) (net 7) (status 10))
 (segment (start 132.024999 124.404999) (end 135.89 128.27) (width 0.2) (layer F.Cu) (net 10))
 (segment (start 123.515001 124.404999) (end 132.024999 124.404999) (width 0.2) (layer F.Cu) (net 10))
 (segment (start 121.92 126) (end 123.515001 124.404999) (width 0.2) (layer F.Cu) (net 10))
 (segment (start 114.03 131.81) (end 114.03 132.4) (width 0.2) (layer F.Cu) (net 3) (status 20))
 (segment (start 113.57 131.35) (end 114.03 131.81) (width 0.2) (layer F.Cu) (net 3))
 (segment (start 109.95 131.35) (end 109.22 132.08) (width 0.2) (layer F.Cu) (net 3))
 (segment (start 113.57 131.35) (end 109.95 131.35) (width 0.2) (layer F.Cu) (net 3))
 (segment (start 105.41 132.08) (end 104.14 133.35) (width 0.2) (layer F.Cu) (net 3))
 (segment (start 109.22 132.08) (end 105.41 132.08) (width 0.2) (layer F.Cu) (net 3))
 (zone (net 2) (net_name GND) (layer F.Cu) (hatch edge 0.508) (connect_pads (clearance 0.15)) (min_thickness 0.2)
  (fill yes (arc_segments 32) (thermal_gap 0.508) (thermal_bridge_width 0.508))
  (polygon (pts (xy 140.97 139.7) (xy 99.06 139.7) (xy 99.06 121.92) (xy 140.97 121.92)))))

